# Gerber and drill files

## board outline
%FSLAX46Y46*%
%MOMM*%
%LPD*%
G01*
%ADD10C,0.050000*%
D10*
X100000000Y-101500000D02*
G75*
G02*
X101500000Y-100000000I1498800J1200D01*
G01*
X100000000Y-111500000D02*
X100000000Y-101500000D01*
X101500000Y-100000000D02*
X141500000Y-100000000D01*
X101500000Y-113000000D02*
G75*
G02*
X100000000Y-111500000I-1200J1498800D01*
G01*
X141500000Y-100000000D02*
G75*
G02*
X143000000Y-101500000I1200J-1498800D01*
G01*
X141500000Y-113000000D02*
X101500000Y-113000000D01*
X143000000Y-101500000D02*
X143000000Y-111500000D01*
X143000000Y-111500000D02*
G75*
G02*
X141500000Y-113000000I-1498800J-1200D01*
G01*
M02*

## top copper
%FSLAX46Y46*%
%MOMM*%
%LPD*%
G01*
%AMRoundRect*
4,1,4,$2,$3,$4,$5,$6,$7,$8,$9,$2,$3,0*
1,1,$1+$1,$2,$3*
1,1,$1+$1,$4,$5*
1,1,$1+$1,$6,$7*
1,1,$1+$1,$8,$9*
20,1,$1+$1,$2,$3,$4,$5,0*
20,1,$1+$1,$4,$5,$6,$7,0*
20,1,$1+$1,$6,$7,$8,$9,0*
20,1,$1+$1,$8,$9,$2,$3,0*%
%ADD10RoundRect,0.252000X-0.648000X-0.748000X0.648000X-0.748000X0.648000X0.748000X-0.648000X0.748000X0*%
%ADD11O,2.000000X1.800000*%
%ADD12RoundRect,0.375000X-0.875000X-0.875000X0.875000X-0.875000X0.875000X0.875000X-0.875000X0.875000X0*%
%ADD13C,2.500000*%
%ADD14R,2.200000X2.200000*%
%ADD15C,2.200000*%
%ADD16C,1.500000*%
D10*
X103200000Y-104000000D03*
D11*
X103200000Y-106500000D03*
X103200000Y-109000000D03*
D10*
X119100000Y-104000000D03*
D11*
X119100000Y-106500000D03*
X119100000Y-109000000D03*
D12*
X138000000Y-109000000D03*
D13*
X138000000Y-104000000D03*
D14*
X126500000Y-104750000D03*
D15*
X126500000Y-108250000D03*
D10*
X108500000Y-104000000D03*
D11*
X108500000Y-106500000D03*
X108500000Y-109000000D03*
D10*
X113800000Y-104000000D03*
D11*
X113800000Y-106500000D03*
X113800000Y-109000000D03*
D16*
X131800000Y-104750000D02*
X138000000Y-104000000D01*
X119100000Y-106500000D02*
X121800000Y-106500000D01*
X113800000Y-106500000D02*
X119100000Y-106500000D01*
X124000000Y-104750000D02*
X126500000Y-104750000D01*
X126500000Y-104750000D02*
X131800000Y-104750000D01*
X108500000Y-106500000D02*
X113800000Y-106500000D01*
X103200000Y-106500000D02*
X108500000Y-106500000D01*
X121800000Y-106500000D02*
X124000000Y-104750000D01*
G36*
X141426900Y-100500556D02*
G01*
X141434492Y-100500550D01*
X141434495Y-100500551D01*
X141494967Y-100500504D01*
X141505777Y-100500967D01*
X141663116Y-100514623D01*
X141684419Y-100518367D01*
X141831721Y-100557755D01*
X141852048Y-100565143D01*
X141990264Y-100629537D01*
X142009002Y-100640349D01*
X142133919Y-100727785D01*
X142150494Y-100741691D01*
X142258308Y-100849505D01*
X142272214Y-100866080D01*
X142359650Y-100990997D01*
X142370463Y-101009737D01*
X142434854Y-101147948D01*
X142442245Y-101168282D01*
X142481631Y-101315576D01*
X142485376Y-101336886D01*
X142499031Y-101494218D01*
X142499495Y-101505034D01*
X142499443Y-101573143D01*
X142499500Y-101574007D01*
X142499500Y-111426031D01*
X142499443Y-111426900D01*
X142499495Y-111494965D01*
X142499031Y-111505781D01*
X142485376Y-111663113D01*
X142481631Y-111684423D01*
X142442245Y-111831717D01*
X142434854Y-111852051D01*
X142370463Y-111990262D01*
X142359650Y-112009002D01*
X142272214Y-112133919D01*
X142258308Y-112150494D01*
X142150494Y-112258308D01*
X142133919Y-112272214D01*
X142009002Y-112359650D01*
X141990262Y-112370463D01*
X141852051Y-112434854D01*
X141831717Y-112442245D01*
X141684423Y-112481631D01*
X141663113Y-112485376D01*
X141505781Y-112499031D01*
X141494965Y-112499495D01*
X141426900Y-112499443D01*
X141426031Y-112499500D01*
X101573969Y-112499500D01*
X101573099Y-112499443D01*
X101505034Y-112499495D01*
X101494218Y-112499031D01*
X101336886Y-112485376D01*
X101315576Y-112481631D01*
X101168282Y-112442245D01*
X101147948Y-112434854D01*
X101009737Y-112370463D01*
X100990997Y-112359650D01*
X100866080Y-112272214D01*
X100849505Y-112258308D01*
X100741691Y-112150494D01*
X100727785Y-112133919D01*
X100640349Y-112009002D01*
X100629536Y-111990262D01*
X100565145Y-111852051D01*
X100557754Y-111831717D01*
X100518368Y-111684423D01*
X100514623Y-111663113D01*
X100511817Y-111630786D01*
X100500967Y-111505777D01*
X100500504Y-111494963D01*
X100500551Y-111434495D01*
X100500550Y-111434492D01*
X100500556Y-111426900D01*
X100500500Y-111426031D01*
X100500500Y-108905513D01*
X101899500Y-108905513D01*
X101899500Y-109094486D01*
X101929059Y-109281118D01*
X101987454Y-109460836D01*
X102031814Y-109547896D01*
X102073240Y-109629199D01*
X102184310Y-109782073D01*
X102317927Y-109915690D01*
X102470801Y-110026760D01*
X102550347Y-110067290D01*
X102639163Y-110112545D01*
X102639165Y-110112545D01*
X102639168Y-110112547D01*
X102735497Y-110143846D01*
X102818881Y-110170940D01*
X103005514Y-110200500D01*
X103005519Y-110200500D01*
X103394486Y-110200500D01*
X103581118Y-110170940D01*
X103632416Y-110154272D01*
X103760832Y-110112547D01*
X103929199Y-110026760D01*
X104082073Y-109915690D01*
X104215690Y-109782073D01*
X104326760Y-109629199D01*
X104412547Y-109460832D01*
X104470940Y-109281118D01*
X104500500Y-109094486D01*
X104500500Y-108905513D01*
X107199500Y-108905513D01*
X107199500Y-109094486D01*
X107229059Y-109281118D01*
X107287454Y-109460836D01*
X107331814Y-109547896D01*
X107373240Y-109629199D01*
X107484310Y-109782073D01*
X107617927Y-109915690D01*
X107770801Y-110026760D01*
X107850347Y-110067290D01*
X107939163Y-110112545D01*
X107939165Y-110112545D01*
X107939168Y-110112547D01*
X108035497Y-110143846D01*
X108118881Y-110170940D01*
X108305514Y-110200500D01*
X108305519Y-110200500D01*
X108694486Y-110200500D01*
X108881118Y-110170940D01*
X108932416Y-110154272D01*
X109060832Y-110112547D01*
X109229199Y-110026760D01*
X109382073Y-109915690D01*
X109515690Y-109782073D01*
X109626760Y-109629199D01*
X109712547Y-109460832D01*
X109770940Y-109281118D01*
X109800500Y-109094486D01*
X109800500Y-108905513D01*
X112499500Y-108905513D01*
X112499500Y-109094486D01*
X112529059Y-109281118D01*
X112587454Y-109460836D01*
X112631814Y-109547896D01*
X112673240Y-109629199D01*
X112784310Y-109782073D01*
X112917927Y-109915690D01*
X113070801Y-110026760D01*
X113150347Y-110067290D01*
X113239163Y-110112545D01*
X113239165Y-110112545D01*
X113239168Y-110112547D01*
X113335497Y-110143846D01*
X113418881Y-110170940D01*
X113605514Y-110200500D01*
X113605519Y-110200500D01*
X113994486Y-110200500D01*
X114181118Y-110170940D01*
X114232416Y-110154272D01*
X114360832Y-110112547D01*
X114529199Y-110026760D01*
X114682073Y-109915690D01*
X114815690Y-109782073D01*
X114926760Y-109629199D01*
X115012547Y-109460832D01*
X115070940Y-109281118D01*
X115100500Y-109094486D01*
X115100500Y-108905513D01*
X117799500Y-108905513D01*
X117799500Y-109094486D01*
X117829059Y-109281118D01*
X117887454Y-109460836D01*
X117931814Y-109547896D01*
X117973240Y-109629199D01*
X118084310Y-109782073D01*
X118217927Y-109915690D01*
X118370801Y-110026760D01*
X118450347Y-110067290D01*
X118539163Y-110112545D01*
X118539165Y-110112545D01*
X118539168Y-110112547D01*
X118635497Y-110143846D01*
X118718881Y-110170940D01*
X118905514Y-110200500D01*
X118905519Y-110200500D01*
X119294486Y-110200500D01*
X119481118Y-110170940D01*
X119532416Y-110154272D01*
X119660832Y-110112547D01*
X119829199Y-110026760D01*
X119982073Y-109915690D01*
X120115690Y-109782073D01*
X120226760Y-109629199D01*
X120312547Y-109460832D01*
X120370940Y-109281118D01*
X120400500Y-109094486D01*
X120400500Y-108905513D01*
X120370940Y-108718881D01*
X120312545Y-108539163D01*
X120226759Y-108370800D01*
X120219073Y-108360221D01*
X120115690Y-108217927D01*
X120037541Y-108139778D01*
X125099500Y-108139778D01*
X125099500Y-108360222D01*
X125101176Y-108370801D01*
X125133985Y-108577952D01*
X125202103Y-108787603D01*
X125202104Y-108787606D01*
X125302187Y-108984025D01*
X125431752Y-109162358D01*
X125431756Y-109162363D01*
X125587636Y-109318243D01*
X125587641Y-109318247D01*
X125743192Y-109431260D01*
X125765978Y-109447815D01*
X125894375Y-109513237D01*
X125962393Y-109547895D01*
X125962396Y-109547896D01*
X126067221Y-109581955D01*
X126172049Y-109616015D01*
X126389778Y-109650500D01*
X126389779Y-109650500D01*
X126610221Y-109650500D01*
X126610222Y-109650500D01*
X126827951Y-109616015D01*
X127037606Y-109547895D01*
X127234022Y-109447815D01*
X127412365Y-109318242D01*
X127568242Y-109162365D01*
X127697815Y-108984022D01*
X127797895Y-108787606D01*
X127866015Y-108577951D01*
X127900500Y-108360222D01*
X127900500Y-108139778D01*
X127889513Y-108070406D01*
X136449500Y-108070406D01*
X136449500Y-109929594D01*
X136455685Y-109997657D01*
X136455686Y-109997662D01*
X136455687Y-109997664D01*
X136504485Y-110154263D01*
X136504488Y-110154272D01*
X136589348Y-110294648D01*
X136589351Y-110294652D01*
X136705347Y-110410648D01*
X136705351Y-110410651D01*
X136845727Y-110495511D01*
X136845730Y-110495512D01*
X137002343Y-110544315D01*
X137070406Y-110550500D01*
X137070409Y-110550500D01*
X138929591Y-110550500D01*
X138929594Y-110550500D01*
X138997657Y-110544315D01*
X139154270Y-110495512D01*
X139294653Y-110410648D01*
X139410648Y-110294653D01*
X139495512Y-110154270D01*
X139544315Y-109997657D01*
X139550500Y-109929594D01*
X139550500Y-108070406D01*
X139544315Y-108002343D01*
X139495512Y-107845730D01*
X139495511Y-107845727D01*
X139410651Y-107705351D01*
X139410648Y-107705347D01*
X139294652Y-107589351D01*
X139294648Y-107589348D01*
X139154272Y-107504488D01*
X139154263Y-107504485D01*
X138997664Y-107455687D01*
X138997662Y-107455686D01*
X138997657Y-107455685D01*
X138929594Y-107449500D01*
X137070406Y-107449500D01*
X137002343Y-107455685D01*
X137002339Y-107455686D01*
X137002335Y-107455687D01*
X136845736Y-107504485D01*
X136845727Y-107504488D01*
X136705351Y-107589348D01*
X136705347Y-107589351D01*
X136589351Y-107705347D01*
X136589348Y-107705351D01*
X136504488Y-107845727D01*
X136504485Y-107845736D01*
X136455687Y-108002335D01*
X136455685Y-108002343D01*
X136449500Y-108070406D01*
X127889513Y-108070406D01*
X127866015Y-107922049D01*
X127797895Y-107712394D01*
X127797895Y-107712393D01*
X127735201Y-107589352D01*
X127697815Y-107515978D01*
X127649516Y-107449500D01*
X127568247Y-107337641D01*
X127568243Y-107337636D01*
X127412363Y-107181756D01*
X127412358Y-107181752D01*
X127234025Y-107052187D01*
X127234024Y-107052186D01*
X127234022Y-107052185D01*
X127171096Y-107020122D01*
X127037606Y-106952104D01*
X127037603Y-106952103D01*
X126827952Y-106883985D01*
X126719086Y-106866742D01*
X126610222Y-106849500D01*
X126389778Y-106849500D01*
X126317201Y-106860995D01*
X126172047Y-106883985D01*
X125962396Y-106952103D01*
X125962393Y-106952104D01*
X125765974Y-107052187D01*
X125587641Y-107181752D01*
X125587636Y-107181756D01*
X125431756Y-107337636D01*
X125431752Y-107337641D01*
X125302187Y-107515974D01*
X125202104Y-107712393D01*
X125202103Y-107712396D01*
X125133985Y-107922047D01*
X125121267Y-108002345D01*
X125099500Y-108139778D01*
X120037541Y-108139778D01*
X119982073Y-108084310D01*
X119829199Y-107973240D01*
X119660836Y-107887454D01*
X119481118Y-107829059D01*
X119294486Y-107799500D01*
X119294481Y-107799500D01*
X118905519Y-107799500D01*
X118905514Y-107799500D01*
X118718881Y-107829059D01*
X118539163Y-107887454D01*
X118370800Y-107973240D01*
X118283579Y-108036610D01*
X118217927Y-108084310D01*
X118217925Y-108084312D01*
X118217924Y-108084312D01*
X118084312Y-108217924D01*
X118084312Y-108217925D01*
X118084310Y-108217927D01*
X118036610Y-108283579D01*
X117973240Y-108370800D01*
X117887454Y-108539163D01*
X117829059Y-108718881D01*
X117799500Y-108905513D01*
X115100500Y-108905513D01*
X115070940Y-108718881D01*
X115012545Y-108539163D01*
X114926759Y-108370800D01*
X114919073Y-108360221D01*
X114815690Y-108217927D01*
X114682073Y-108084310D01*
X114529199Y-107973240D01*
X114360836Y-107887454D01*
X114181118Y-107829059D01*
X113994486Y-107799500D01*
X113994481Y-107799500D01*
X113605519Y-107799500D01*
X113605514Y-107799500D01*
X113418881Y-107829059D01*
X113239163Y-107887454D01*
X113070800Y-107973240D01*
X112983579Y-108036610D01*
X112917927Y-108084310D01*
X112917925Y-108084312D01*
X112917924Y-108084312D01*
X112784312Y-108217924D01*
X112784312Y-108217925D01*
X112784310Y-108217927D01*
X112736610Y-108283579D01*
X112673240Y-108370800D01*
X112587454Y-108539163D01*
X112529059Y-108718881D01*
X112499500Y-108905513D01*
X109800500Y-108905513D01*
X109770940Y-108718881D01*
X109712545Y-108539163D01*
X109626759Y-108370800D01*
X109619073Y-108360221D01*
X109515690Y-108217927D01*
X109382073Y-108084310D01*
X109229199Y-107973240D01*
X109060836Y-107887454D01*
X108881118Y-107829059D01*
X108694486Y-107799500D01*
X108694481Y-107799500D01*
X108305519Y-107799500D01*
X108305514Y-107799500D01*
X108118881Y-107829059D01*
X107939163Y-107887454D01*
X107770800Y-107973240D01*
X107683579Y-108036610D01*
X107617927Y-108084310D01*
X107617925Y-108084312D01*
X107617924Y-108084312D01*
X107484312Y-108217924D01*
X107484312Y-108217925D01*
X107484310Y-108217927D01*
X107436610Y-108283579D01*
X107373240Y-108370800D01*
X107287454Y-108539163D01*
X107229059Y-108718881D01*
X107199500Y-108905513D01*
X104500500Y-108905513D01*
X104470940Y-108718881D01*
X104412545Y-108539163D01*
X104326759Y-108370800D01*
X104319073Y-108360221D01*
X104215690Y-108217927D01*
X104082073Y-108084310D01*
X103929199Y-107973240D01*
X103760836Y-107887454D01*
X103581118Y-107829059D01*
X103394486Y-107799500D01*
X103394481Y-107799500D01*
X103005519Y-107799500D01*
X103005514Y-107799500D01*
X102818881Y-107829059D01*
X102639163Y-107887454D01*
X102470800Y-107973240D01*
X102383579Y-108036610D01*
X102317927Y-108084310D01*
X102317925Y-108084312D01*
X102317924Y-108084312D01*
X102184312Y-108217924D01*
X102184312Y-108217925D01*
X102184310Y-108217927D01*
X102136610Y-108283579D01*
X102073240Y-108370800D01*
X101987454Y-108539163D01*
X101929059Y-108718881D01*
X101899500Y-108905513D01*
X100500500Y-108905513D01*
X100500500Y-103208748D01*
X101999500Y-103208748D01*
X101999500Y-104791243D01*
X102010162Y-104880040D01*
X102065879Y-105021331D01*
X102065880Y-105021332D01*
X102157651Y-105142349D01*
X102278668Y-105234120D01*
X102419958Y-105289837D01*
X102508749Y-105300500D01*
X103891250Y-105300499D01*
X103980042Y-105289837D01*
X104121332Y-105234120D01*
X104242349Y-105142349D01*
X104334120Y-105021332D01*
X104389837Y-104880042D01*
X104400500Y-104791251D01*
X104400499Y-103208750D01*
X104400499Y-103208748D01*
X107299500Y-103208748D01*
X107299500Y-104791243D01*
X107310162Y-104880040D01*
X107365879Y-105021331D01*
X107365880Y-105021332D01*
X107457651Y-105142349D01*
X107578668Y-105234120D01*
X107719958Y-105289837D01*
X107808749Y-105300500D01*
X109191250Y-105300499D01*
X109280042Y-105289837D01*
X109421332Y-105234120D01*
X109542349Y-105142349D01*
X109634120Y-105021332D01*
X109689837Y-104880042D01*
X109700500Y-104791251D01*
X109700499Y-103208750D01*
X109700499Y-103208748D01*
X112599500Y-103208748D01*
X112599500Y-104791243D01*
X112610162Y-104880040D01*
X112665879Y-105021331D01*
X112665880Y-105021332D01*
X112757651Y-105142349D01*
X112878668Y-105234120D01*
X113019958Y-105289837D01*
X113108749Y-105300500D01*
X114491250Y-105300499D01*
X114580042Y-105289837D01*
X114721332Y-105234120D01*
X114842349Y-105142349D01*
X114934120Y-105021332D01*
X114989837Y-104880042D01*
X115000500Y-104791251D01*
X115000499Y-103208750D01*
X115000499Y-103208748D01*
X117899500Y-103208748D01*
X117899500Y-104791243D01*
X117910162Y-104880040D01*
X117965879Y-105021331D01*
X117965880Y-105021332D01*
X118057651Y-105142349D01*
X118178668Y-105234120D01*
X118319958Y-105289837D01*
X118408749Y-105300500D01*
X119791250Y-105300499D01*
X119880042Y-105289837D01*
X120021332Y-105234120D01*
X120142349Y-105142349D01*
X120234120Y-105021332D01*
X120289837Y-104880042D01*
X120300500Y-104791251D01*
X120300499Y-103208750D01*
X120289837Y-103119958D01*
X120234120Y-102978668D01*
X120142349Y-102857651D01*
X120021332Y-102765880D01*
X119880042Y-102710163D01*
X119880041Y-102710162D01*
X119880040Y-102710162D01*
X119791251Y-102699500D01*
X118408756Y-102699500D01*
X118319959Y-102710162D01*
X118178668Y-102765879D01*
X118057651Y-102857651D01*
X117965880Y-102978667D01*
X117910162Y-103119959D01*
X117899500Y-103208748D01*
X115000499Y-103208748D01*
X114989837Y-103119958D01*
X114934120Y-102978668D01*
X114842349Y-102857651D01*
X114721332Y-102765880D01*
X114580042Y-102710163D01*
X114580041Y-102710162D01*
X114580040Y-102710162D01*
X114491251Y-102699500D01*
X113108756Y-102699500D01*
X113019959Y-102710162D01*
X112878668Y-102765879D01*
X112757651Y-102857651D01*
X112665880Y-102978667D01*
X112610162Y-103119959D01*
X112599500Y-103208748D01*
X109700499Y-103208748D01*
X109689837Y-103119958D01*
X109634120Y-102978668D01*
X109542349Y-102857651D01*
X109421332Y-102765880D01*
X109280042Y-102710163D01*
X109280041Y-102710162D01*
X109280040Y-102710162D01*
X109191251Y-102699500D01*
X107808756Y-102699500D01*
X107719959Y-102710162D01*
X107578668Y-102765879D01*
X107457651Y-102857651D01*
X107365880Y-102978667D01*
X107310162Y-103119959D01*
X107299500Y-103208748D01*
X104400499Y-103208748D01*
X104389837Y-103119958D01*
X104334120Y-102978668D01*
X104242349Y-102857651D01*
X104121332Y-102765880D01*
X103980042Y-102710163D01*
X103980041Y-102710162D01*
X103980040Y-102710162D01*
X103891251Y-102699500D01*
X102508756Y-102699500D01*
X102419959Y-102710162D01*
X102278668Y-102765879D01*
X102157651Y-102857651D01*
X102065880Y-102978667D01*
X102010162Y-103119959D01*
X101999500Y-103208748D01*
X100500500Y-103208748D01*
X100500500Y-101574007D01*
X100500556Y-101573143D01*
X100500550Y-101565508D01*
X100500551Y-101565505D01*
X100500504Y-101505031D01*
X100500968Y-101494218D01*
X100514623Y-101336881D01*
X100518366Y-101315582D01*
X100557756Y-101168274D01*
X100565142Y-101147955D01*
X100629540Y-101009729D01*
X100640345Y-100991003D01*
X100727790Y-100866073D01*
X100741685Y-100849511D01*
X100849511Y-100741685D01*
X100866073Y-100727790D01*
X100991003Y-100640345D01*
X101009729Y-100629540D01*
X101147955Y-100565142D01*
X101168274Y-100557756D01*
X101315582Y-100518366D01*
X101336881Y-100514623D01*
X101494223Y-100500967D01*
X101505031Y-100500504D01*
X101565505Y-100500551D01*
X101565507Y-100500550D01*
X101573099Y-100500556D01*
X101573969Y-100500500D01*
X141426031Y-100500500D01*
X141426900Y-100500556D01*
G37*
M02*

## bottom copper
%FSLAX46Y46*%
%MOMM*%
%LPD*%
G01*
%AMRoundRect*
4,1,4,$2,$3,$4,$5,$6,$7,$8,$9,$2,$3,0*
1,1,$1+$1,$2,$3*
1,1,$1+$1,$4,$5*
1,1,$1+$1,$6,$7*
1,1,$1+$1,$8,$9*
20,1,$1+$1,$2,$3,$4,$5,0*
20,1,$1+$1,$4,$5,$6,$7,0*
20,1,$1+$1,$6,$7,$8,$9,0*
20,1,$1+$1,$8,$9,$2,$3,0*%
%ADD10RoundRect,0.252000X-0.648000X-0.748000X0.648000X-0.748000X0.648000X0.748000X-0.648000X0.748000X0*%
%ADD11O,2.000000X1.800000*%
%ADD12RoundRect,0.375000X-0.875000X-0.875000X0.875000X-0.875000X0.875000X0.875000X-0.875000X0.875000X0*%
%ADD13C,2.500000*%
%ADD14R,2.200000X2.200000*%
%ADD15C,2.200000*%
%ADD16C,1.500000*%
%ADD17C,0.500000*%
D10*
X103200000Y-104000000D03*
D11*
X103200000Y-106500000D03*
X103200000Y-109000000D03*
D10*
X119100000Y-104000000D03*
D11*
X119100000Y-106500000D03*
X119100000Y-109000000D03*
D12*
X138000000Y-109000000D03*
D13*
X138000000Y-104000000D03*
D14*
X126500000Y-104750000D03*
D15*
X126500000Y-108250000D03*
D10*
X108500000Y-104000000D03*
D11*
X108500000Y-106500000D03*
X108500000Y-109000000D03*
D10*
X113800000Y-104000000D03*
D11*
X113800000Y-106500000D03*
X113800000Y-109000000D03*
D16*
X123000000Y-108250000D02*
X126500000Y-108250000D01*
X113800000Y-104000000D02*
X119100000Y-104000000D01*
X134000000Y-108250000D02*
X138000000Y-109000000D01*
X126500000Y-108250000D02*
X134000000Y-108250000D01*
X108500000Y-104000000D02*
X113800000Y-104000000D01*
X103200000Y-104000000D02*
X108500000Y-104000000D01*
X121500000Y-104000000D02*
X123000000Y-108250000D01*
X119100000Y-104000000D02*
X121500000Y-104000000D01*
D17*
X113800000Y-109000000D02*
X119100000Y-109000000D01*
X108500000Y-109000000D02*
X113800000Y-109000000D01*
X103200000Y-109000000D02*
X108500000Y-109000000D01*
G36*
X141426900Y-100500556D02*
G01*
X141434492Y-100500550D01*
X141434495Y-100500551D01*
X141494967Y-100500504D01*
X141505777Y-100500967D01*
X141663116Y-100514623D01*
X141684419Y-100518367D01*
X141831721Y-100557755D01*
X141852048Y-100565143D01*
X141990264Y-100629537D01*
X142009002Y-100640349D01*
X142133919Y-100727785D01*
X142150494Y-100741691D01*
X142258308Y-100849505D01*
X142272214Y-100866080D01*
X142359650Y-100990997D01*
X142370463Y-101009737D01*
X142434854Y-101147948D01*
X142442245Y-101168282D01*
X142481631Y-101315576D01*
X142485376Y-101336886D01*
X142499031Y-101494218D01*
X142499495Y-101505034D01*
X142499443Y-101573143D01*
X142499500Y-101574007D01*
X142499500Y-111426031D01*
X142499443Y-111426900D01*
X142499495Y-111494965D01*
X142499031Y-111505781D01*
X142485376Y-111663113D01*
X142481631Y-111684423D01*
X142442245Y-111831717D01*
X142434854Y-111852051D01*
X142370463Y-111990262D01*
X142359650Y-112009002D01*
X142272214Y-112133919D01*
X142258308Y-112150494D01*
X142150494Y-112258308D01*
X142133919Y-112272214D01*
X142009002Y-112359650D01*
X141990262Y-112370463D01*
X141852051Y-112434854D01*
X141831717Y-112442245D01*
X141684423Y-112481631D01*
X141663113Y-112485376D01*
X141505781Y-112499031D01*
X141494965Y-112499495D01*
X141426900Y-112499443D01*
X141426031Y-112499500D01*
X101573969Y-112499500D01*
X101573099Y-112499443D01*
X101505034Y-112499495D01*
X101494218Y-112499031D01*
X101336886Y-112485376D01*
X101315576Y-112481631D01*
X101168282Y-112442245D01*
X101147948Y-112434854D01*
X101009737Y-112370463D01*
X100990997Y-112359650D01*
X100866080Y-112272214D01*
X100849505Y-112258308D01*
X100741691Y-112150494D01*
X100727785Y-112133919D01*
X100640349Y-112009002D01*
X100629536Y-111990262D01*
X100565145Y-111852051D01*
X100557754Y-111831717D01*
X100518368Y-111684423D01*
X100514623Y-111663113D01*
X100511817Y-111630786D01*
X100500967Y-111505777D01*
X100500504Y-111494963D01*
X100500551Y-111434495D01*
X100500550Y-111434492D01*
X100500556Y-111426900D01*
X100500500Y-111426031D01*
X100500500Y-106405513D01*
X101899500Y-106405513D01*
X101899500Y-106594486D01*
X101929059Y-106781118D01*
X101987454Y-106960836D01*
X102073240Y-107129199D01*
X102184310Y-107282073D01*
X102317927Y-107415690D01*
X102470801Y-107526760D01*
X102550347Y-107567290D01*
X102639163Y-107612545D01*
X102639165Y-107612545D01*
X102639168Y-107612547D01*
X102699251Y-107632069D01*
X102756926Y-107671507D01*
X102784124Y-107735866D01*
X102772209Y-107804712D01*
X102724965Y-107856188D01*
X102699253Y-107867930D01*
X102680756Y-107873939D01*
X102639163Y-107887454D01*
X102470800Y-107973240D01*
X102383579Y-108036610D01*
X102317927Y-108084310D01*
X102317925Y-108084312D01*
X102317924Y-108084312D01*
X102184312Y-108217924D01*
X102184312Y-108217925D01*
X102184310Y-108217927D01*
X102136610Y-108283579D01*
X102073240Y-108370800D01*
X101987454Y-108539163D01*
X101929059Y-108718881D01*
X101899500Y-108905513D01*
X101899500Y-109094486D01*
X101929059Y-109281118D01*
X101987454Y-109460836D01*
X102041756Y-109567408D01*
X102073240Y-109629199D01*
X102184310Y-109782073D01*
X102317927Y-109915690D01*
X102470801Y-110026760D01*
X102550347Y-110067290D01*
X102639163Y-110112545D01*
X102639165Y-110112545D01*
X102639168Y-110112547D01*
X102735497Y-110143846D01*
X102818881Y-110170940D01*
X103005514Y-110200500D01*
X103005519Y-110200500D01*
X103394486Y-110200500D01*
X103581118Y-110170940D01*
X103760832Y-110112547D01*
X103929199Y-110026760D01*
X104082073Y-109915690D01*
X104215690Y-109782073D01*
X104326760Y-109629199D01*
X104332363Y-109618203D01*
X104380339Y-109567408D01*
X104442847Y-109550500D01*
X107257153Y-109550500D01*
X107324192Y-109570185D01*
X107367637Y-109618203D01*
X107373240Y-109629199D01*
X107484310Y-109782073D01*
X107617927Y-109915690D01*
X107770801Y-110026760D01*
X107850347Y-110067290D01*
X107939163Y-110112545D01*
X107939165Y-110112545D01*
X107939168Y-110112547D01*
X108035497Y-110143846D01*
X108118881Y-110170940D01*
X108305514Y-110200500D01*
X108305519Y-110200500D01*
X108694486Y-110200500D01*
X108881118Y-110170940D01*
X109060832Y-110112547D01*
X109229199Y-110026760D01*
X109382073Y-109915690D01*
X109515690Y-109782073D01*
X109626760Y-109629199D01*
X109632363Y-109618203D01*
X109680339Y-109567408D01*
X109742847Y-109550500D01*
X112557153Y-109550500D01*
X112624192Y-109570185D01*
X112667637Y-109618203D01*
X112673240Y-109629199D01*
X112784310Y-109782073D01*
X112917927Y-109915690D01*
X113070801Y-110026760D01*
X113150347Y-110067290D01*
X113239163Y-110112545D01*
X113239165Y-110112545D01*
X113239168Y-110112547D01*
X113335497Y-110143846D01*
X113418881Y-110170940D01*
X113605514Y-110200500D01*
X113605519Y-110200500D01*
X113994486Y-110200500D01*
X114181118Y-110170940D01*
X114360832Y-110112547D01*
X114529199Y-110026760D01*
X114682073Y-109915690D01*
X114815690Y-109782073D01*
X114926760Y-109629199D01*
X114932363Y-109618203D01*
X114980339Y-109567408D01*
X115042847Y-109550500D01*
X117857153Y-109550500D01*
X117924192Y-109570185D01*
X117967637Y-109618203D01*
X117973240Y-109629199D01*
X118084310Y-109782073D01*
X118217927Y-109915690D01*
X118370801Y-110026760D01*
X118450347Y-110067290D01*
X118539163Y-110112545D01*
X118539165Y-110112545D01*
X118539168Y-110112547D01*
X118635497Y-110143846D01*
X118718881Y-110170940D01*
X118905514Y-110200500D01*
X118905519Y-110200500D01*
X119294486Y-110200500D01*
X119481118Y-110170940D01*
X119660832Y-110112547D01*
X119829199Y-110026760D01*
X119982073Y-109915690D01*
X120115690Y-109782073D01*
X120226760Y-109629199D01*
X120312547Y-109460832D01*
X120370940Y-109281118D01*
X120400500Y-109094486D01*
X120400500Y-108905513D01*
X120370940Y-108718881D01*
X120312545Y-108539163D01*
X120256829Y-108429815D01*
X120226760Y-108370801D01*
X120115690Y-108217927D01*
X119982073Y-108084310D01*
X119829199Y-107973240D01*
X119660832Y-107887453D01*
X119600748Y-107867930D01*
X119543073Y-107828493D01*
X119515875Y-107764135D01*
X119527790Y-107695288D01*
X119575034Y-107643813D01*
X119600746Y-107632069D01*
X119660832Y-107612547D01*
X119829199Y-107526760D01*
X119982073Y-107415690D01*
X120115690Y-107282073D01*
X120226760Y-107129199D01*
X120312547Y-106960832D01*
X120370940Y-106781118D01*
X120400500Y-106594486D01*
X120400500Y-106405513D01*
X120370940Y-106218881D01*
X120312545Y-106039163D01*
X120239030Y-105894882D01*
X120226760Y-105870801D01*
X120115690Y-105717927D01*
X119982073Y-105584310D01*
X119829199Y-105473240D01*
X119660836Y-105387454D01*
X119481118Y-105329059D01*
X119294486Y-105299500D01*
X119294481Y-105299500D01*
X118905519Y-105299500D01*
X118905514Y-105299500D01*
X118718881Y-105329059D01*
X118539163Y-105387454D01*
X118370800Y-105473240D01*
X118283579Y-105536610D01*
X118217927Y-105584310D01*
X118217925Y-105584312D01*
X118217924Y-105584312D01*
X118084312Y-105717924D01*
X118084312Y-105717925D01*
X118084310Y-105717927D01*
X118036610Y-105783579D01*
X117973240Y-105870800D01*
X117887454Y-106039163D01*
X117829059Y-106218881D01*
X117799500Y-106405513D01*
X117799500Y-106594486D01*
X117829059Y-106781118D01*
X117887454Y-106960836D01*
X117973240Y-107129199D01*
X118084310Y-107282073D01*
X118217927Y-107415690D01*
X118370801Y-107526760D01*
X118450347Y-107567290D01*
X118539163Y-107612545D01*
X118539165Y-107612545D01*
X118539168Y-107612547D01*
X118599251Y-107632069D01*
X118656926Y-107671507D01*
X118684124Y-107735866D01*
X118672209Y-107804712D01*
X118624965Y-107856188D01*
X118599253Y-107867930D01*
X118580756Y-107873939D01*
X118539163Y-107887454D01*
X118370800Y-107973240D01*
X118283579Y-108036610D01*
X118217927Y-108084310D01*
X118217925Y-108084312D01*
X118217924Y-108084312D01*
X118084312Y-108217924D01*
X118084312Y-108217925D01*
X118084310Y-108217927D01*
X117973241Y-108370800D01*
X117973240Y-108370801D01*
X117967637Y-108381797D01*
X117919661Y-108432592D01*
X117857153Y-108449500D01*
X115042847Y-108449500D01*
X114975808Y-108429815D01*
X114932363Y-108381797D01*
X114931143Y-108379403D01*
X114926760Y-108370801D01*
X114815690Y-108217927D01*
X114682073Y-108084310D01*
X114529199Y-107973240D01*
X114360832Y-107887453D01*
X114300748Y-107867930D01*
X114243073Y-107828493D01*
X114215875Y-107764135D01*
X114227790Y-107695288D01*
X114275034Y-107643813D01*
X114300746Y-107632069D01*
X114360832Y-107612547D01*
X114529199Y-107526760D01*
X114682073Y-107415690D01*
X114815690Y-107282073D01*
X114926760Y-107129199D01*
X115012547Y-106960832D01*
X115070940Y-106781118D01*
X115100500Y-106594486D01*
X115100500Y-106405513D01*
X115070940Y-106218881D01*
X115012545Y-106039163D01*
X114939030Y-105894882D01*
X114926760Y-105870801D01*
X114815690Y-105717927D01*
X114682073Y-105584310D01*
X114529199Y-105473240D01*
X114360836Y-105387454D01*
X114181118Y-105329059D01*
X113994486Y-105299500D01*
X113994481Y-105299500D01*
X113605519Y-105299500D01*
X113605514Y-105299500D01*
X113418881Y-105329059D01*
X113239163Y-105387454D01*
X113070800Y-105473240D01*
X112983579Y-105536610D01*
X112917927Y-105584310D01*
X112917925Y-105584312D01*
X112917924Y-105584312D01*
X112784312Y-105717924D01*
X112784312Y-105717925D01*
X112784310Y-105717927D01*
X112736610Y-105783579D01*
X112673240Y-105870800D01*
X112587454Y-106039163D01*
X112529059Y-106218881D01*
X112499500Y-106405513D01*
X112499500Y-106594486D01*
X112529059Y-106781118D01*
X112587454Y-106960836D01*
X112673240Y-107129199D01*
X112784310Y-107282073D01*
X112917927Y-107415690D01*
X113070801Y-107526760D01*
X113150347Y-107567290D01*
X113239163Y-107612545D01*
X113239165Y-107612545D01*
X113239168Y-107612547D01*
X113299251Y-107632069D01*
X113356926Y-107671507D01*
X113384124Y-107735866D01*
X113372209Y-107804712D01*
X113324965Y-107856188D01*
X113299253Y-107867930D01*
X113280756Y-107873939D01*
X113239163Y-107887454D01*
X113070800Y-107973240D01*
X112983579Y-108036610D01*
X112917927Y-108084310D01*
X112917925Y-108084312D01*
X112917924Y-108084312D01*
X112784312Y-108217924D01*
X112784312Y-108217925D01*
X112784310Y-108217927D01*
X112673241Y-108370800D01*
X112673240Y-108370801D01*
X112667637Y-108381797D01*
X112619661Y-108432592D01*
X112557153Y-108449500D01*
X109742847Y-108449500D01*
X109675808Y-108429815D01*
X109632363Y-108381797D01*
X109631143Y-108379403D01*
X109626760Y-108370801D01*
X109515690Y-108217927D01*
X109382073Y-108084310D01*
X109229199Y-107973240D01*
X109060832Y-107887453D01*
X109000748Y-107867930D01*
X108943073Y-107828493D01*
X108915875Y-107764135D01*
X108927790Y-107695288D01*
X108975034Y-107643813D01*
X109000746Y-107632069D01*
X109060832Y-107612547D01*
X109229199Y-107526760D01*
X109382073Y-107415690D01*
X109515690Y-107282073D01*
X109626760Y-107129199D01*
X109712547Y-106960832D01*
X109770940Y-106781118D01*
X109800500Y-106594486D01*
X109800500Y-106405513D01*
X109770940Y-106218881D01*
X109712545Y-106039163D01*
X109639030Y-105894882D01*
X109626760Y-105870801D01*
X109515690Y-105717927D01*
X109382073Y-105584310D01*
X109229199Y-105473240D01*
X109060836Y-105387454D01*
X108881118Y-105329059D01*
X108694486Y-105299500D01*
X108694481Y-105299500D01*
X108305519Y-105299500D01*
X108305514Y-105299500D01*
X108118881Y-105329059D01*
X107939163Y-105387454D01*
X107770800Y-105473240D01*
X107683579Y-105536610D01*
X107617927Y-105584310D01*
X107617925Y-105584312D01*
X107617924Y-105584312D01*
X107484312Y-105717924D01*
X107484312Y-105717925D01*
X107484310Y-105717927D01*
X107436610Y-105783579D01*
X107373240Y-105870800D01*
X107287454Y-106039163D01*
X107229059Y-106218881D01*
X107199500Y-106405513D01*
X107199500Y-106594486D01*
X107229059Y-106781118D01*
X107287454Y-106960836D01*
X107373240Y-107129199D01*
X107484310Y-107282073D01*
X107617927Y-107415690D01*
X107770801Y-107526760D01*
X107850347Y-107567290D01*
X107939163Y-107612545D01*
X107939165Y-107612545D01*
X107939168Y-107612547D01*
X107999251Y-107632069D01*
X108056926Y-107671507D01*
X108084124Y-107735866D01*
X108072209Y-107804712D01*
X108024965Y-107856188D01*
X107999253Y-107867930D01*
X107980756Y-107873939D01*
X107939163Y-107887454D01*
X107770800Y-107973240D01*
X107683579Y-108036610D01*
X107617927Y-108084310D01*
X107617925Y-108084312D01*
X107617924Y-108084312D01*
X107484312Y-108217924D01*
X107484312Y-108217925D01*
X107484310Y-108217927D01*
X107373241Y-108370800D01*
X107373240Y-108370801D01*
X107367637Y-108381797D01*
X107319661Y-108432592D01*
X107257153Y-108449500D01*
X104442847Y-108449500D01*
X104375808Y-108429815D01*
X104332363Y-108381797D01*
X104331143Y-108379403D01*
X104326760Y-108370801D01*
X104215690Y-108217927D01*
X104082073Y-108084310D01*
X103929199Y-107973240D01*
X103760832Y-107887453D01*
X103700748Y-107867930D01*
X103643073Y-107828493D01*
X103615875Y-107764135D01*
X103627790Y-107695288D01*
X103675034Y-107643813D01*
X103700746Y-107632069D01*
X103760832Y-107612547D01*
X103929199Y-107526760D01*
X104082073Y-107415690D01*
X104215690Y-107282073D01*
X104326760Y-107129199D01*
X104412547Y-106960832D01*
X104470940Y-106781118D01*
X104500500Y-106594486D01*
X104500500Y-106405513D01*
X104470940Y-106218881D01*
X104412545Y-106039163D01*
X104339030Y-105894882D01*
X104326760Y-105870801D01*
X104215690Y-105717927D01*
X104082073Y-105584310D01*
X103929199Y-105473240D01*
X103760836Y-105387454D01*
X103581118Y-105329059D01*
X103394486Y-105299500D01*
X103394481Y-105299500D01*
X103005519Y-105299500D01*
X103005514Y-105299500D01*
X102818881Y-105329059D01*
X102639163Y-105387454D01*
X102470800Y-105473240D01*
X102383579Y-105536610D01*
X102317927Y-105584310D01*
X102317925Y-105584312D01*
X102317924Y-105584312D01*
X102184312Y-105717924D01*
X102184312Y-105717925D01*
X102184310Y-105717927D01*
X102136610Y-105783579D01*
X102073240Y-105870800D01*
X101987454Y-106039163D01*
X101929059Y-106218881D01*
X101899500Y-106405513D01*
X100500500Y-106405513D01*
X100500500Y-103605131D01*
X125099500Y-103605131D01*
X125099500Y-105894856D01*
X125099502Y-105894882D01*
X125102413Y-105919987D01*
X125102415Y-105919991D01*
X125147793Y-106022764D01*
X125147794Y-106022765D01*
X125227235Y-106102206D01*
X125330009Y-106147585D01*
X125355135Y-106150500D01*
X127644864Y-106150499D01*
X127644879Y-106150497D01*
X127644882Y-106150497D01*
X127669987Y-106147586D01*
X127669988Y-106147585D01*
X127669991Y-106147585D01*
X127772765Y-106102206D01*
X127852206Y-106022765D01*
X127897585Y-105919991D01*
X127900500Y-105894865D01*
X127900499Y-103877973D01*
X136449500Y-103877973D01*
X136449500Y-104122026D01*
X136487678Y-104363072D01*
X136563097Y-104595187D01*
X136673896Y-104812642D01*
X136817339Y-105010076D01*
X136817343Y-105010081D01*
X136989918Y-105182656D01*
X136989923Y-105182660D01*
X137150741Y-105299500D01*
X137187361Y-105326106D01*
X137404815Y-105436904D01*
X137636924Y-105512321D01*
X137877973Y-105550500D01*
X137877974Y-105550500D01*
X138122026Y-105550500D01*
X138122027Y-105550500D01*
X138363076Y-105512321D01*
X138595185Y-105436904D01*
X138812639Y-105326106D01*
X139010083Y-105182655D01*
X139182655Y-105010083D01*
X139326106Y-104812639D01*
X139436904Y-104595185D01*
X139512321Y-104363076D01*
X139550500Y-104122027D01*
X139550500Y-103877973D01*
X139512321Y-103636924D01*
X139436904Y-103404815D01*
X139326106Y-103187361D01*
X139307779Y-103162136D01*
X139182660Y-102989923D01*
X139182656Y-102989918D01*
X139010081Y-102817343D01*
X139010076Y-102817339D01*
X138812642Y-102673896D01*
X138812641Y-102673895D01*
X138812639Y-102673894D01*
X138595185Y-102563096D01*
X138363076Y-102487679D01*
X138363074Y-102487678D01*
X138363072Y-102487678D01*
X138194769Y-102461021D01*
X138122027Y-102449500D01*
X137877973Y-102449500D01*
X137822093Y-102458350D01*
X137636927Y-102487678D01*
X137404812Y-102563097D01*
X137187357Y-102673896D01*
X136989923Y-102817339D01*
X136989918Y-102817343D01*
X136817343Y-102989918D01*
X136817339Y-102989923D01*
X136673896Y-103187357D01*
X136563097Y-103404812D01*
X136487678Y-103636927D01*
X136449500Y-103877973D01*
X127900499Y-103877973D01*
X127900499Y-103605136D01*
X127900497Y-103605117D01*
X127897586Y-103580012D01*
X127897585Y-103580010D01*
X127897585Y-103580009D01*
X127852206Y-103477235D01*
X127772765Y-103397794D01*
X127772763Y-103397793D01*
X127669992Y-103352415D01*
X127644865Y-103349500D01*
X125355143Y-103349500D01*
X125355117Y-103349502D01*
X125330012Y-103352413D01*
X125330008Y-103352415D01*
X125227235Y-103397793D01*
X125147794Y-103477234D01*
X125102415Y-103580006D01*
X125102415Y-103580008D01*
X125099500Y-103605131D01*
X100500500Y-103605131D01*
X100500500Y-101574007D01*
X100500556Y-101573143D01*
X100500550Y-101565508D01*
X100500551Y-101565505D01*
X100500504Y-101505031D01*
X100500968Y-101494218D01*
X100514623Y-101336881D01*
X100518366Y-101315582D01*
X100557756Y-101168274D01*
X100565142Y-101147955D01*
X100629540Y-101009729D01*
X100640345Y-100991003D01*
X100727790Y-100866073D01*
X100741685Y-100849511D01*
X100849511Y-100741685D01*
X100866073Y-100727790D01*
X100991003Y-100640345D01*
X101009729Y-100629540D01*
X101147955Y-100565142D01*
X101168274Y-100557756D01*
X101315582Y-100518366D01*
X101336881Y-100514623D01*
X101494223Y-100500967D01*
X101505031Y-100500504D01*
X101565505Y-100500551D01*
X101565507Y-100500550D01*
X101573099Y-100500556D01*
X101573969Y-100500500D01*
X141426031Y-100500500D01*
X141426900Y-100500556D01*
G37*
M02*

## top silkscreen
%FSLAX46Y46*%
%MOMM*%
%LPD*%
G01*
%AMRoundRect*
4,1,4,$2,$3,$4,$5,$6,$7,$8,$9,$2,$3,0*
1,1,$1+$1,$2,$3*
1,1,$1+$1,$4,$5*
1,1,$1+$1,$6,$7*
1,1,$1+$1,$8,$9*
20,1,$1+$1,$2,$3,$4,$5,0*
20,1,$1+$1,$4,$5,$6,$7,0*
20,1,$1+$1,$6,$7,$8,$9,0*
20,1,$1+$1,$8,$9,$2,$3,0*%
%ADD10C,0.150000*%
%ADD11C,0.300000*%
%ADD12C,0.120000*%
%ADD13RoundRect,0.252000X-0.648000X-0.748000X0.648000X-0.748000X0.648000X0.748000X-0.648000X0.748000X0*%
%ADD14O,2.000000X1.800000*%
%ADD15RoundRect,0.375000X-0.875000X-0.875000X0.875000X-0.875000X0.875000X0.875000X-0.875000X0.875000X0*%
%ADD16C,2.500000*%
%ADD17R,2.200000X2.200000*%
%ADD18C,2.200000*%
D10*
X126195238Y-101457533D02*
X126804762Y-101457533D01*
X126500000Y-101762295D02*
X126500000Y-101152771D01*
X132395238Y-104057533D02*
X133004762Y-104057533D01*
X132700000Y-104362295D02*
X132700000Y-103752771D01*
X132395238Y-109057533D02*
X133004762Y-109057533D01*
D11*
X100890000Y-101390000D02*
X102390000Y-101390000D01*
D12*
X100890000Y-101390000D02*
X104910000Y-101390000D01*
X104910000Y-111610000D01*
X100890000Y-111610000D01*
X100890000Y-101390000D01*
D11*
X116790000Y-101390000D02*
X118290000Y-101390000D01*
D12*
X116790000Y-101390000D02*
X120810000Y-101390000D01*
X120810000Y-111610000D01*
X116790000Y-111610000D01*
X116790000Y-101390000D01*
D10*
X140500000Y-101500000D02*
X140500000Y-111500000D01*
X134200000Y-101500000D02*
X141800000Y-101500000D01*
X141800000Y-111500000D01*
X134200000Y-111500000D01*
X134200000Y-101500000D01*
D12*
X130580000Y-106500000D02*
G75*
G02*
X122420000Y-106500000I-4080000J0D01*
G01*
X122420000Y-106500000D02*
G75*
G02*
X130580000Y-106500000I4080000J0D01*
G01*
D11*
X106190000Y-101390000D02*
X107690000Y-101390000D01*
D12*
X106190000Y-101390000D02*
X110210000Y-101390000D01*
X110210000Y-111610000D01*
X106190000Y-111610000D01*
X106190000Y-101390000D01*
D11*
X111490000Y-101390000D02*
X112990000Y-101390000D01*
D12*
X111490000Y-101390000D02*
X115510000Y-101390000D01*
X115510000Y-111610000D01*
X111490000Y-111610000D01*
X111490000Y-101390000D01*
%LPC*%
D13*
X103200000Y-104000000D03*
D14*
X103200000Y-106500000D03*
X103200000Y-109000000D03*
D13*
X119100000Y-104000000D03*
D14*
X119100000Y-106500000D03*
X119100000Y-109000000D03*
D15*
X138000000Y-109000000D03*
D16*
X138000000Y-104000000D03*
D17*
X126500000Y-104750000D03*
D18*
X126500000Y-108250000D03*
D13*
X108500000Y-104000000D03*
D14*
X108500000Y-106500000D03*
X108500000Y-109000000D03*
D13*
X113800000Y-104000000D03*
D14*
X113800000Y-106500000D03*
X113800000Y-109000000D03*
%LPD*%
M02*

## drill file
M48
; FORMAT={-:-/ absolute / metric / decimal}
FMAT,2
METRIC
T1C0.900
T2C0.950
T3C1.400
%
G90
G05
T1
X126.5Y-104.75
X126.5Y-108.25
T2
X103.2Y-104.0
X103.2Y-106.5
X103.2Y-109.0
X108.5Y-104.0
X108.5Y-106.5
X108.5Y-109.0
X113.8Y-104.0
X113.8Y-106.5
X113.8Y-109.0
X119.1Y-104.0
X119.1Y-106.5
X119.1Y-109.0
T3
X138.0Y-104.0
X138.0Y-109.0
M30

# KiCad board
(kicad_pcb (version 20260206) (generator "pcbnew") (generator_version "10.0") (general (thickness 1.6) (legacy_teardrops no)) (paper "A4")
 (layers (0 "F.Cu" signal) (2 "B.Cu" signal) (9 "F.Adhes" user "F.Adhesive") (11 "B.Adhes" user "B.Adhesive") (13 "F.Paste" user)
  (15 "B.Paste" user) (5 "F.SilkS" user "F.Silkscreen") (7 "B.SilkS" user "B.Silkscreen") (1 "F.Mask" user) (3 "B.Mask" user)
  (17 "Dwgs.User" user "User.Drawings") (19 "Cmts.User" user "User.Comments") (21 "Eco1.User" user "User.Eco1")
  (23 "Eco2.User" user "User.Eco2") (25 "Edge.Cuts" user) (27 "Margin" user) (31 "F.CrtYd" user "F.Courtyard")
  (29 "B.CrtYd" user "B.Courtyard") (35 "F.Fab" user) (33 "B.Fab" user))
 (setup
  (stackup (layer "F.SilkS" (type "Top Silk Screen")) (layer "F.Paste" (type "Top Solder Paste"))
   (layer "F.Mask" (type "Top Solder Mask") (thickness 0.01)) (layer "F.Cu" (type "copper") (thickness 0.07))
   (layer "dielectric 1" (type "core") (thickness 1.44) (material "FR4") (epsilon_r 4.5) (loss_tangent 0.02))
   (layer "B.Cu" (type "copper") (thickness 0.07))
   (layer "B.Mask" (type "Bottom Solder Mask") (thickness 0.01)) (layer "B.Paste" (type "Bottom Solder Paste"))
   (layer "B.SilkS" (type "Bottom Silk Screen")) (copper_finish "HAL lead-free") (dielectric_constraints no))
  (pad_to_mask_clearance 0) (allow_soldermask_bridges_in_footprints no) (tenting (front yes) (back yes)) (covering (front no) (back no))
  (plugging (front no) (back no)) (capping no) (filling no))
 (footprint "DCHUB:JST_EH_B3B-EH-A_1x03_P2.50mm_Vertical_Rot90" (layer "F.Cu") (at 103.2 104)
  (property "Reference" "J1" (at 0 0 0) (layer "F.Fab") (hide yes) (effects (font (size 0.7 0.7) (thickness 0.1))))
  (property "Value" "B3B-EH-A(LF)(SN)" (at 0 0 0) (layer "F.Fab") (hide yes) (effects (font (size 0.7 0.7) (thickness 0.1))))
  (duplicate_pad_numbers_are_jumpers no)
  (fp_line (start -2.31 -2.61) (end -0.81 -2.61) (stroke (width 0.3) (type solid)) (layer "F.SilkS"))
  (fp_rect (start -2.31 -2.61) (end 1.71 7.61) (stroke (width 0.12) (type solid)) (fill no) (layer "F.SilkS"))
  (pad "1" thru_hole roundrect (at 0 0) (size 1.8 2) (drill 0.95) (layers "*.Cu" "*.Mask") (remove_unused_layers no) (roundrect_rratio 0.14)
   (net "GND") (zone_connect 2))
  (pad "2" thru_hole oval (at 0 2.5) (size 2 1.8) (drill 0.95) (layers "*.Cu" "*.Mask") (remove_unused_layers no) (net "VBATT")
   (zone_connect 2))
  (pad "3" thru_hole oval (at 0 5) (size 2 1.8) (drill 0.95) (layers "*.Cu" "*.Mask") (remove_unused_layers no) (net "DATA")))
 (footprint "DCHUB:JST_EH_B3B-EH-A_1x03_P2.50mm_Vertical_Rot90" (layer "F.Cu") (at 119.1 104)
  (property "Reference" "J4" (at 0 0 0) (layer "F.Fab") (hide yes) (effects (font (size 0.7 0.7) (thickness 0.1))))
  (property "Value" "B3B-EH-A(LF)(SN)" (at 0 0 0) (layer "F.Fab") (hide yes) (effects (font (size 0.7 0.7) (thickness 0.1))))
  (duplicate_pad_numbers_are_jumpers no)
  (fp_line (start -2.31 -2.61) (end -0.81 -2.61) (stroke (width 0.3) (type solid)) (layer "F.SilkS"))
  (fp_rect (start -2.31 -2.61) (end 1.71 7.61) (stroke (width 0.12) (type solid)) (fill no) (layer "F.SilkS"))
  (pad "1" thru_hole roundrect (at 0 0) (size 1.8 2) (drill 0.95) (layers "*.Cu" "*.Mask") (remove_unused_layers no) (roundrect_rratio 0.14)
   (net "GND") (zone_connect 2))
  (pad "2" thru_hole oval (at 0 2.5) (size 2 1.8) (drill 0.95) (layers "*.Cu" "*.Mask") (remove_unused_layers no) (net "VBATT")
   (zone_connect 2))
  (pad "3" thru_hole oval (at 0 5) (size 2 1.8) (drill 0.95) (layers "*.Cu" "*.Mask") (remove_unused_layers no) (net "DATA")))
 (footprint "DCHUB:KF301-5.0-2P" (layer "F.Cu") (at 138 106.5)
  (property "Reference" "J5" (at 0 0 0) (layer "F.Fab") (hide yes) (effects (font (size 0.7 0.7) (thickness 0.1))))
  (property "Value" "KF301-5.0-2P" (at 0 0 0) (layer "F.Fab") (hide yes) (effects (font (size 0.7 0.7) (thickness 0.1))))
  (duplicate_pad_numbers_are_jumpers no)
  (fp_line (start 2.5 -5) (end 2.5 5) (stroke (width 0.15) (type solid)) (layer "F.SilkS"))
  (fp_rect (start -3.8 -5) (end 3.8 5) (stroke (width 0.15) (type solid)) (fill no) (layer "F.SilkS"))
  (pad "1" thru_hole roundrect (at 0 2.5) (size 2.5 2.5) (drill 1.4) (layers "*.Cu" "*.Mask") (remove_unused_layers no)
   (roundrect_rratio 0.15) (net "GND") (zone_connect 2))
  (pad "2" thru_hole circle (at 0 -2.5) (size 2.5 2.5) (drill 1.4) (layers "*.Cu" "*.Mask") (remove_unused_layers no) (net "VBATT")
   (zone_connect 2)))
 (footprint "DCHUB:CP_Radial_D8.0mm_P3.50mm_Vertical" (layer "F.Cu") (at 126.5 104.75)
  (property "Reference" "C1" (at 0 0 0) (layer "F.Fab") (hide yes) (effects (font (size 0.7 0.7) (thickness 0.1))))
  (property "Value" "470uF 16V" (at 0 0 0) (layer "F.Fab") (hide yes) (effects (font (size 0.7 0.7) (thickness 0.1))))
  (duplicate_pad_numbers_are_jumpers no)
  (fp_circle (center 0 1.75) (end 4.08 1.75) (stroke (width 0.12) (type solid)) (fill no) (layer "F.SilkS"))
  (pad "1" thru_hole rect (at 0 0) (size 2.2 2.2) (drill 0.9) (layers "*.Cu" "*.Mask") (remove_unused_layers no) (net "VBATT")
   (zone_connect 2))
  (pad "2" thru_hole circle (at 0 3.5) (size 2.2 2.2) (drill 0.9) (layers "*.Cu" "*.Mask") (remove_unused_layers no) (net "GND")
   (zone_connect 2)))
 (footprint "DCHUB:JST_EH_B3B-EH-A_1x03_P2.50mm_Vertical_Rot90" (layer "F.Cu") (at 108.5 104)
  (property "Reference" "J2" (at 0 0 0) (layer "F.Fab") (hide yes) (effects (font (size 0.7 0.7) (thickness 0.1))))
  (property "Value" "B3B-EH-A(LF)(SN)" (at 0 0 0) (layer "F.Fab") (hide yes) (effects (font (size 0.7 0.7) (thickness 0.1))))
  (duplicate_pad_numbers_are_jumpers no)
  (fp_line (start -2.31 -2.61) (end -0.81 -2.61) (stroke (width 0.3) (type solid)) (layer "F.SilkS"))
  (fp_rect (start -2.31 -2.61) (end 1.71 7.61) (stroke (width 0.12) (type solid)) (fill no) (layer "F.SilkS"))
  (pad "1" thru_hole roundrect (at 0 0) (size 1.8 2) (drill 0.95) (layers "*.Cu" "*.Mask") (remove_unused_layers no) (roundrect_rratio 0.14)
   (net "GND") (zone_connect 2))
  (pad "2" thru_hole oval (at 0 2.5) (size 2 1.8) (drill 0.95) (layers "*.Cu" "*.Mask") (remove_unused_layers no) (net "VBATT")
   (zone_connect 2))
  (pad "3" thru_hole oval (at 0 5) (size 2 1.8) (drill 0.95) (layers "*.Cu" "*.Mask") (remove_unused_layers no) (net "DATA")))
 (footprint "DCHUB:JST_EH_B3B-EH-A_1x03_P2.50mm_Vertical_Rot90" (layer "F.Cu") (at 113.8 104)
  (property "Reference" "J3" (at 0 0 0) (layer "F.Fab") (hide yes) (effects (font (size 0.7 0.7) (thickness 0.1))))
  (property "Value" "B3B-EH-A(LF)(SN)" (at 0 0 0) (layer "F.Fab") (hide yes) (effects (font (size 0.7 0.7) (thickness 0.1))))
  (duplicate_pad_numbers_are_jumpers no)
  (fp_line (start -2.31 -2.61) (end -0.81 -2.61) (stroke (width 0.3) (type solid)) (layer "F.SilkS"))
  (fp_rect (start -2.31 -2.61) (end 1.71 7.61) (stroke (width 0.12) (type solid)) (fill no) (layer "F.SilkS"))
  (pad "1" thru_hole roundrect (at 0 0) (size 1.8 2) (drill 0.95) (layers "*.Cu" "*.Mask") (remove_unused_layers no) (roundrect_rratio 0.14)
   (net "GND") (zone_connect 2))
  (pad "2" thru_hole oval (at 0 2.5) (size 2 1.8) (drill 0.95) (layers "*.Cu" "*.Mask") (remove_unused_layers no) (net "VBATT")
   (zone_connect 2))
  (pad "3" thru_hole oval (at 0 5) (size 2 1.8) (drill 0.95) (layers "*.Cu" "*.Mask") (remove_unused_layers no) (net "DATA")))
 (gr_arc (start 100 101.5) (mid 100.439 100.439) (end 101.5 100) (stroke (width 0.05) (type solid)) (layer "Edge.Cuts"))
 (gr_line (start 100 111.5) (end 100 101.5) (stroke (width 0.05) (type solid)) (layer "Edge.Cuts"))
 (gr_line (start 101.5 100) (end 141.5 100) (stroke (width 0.05) (type solid)) (layer "Edge.Cuts"))
 (gr_arc (start 101.5 113) (mid 100.439 112.561) (end 100 111.5) (stroke (width 0.05) (type solid)) (layer "Edge.Cuts"))
 (gr_arc (start 141.5 100) (mid 142.561 100.439) (end 143 101.5) (stroke (width 0.05) (type solid)) (layer "Edge.Cuts"))
 (gr_line (start 141.5 113) (end 101.5 113) (stroke (width 0.05) (type solid)) (layer "Edge.Cuts"))
 (gr_line (start 143 101.5) (end 143 111.5) (stroke (width 0.05) (type solid)) (layer "Edge.Cuts"))
 (gr_arc (start 143 111.5) (mid 142.561 112.561) (end 141.5 113) (stroke (width 0.05) (type solid)) (layer "Edge.Cuts"))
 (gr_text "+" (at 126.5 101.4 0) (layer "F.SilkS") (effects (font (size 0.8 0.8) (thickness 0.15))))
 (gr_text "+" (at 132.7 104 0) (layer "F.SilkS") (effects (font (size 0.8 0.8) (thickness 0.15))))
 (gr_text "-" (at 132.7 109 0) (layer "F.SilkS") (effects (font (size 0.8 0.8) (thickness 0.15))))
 (segment (start 123 108.25) (end 126.5 108.25) (width 1.5) (layer "B.Cu") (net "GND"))
 (segment (start 113.8 104) (end 119.1 104) (width 1.5) (layer "B.Cu") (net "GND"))
 (segment (start 134 108.25) (end 138 109) (width 1.5) (layer "B.Cu") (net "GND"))
 (segment (start 126.5 108.25) (end 134 108.25) (width 1.5) (layer "B.Cu") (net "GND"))
 (segment (start 108.5 104) (end 113.8 104) (width 1.5) (layer "B.Cu") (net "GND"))
 (segment (start 103.2 104) (end 108.5 104) (width 1.5) (layer "B.Cu") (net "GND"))
 (segment (start 121.5 104) (end 123 108.25) (width 1.5) (layer "B.Cu") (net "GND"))
 (segment (start 119.1 104) (end 121.5 104) (width 1.5) (layer "B.Cu") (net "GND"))
 (segment (start 131.8 104.75) (end 138 104) (width 1.5) (layer "F.Cu") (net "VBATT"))
 (segment (start 119.1 106.5) (end 121.8 106.5) (width 1.5) (layer "F.Cu") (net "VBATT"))
 (segment (start 113.8 106.5) (end 119.1 106.5) (width 1.5) (layer "F.Cu") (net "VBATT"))
 (segment (start 124 104.75) (end 126.5 104.75) (width 1.5) (layer "F.Cu") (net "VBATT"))
 (segment (start 126.5 104.75) (end 131.8 104.75) (width 1.5) (layer "F.Cu") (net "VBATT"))
 (segment (start 108.5 106.5) (end 113.8 106.5) (width 1.5) (layer "F.Cu") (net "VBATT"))
 (segment (start 103.2 106.5) (end 108.5 106.5) (width 1.5) (layer "F.Cu") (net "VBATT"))
 (segment (start 121.8 106.5) (end 124 104.75) (width 1.5) (layer "F.Cu") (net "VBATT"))
 (segment (start 113.8 109) (end 119.1 109) (width 0.5) (layer "B.Cu") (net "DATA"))
 (segment (start 108.5 109) (end 113.8 109) (width 0.5) (layer "B.Cu") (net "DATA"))
 (segment (start 103.2 109) (end 108.5 109) (width 0.5) (layer "B.Cu") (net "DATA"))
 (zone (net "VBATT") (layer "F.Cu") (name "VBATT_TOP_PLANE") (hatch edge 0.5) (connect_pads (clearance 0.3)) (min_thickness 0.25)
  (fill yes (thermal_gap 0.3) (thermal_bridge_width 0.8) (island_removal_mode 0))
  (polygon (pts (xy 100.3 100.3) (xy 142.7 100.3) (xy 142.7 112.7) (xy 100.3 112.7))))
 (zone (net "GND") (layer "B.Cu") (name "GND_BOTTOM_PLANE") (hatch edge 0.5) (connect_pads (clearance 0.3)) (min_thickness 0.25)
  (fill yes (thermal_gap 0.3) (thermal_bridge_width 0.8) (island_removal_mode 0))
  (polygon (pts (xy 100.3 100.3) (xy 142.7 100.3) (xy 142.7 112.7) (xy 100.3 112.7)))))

